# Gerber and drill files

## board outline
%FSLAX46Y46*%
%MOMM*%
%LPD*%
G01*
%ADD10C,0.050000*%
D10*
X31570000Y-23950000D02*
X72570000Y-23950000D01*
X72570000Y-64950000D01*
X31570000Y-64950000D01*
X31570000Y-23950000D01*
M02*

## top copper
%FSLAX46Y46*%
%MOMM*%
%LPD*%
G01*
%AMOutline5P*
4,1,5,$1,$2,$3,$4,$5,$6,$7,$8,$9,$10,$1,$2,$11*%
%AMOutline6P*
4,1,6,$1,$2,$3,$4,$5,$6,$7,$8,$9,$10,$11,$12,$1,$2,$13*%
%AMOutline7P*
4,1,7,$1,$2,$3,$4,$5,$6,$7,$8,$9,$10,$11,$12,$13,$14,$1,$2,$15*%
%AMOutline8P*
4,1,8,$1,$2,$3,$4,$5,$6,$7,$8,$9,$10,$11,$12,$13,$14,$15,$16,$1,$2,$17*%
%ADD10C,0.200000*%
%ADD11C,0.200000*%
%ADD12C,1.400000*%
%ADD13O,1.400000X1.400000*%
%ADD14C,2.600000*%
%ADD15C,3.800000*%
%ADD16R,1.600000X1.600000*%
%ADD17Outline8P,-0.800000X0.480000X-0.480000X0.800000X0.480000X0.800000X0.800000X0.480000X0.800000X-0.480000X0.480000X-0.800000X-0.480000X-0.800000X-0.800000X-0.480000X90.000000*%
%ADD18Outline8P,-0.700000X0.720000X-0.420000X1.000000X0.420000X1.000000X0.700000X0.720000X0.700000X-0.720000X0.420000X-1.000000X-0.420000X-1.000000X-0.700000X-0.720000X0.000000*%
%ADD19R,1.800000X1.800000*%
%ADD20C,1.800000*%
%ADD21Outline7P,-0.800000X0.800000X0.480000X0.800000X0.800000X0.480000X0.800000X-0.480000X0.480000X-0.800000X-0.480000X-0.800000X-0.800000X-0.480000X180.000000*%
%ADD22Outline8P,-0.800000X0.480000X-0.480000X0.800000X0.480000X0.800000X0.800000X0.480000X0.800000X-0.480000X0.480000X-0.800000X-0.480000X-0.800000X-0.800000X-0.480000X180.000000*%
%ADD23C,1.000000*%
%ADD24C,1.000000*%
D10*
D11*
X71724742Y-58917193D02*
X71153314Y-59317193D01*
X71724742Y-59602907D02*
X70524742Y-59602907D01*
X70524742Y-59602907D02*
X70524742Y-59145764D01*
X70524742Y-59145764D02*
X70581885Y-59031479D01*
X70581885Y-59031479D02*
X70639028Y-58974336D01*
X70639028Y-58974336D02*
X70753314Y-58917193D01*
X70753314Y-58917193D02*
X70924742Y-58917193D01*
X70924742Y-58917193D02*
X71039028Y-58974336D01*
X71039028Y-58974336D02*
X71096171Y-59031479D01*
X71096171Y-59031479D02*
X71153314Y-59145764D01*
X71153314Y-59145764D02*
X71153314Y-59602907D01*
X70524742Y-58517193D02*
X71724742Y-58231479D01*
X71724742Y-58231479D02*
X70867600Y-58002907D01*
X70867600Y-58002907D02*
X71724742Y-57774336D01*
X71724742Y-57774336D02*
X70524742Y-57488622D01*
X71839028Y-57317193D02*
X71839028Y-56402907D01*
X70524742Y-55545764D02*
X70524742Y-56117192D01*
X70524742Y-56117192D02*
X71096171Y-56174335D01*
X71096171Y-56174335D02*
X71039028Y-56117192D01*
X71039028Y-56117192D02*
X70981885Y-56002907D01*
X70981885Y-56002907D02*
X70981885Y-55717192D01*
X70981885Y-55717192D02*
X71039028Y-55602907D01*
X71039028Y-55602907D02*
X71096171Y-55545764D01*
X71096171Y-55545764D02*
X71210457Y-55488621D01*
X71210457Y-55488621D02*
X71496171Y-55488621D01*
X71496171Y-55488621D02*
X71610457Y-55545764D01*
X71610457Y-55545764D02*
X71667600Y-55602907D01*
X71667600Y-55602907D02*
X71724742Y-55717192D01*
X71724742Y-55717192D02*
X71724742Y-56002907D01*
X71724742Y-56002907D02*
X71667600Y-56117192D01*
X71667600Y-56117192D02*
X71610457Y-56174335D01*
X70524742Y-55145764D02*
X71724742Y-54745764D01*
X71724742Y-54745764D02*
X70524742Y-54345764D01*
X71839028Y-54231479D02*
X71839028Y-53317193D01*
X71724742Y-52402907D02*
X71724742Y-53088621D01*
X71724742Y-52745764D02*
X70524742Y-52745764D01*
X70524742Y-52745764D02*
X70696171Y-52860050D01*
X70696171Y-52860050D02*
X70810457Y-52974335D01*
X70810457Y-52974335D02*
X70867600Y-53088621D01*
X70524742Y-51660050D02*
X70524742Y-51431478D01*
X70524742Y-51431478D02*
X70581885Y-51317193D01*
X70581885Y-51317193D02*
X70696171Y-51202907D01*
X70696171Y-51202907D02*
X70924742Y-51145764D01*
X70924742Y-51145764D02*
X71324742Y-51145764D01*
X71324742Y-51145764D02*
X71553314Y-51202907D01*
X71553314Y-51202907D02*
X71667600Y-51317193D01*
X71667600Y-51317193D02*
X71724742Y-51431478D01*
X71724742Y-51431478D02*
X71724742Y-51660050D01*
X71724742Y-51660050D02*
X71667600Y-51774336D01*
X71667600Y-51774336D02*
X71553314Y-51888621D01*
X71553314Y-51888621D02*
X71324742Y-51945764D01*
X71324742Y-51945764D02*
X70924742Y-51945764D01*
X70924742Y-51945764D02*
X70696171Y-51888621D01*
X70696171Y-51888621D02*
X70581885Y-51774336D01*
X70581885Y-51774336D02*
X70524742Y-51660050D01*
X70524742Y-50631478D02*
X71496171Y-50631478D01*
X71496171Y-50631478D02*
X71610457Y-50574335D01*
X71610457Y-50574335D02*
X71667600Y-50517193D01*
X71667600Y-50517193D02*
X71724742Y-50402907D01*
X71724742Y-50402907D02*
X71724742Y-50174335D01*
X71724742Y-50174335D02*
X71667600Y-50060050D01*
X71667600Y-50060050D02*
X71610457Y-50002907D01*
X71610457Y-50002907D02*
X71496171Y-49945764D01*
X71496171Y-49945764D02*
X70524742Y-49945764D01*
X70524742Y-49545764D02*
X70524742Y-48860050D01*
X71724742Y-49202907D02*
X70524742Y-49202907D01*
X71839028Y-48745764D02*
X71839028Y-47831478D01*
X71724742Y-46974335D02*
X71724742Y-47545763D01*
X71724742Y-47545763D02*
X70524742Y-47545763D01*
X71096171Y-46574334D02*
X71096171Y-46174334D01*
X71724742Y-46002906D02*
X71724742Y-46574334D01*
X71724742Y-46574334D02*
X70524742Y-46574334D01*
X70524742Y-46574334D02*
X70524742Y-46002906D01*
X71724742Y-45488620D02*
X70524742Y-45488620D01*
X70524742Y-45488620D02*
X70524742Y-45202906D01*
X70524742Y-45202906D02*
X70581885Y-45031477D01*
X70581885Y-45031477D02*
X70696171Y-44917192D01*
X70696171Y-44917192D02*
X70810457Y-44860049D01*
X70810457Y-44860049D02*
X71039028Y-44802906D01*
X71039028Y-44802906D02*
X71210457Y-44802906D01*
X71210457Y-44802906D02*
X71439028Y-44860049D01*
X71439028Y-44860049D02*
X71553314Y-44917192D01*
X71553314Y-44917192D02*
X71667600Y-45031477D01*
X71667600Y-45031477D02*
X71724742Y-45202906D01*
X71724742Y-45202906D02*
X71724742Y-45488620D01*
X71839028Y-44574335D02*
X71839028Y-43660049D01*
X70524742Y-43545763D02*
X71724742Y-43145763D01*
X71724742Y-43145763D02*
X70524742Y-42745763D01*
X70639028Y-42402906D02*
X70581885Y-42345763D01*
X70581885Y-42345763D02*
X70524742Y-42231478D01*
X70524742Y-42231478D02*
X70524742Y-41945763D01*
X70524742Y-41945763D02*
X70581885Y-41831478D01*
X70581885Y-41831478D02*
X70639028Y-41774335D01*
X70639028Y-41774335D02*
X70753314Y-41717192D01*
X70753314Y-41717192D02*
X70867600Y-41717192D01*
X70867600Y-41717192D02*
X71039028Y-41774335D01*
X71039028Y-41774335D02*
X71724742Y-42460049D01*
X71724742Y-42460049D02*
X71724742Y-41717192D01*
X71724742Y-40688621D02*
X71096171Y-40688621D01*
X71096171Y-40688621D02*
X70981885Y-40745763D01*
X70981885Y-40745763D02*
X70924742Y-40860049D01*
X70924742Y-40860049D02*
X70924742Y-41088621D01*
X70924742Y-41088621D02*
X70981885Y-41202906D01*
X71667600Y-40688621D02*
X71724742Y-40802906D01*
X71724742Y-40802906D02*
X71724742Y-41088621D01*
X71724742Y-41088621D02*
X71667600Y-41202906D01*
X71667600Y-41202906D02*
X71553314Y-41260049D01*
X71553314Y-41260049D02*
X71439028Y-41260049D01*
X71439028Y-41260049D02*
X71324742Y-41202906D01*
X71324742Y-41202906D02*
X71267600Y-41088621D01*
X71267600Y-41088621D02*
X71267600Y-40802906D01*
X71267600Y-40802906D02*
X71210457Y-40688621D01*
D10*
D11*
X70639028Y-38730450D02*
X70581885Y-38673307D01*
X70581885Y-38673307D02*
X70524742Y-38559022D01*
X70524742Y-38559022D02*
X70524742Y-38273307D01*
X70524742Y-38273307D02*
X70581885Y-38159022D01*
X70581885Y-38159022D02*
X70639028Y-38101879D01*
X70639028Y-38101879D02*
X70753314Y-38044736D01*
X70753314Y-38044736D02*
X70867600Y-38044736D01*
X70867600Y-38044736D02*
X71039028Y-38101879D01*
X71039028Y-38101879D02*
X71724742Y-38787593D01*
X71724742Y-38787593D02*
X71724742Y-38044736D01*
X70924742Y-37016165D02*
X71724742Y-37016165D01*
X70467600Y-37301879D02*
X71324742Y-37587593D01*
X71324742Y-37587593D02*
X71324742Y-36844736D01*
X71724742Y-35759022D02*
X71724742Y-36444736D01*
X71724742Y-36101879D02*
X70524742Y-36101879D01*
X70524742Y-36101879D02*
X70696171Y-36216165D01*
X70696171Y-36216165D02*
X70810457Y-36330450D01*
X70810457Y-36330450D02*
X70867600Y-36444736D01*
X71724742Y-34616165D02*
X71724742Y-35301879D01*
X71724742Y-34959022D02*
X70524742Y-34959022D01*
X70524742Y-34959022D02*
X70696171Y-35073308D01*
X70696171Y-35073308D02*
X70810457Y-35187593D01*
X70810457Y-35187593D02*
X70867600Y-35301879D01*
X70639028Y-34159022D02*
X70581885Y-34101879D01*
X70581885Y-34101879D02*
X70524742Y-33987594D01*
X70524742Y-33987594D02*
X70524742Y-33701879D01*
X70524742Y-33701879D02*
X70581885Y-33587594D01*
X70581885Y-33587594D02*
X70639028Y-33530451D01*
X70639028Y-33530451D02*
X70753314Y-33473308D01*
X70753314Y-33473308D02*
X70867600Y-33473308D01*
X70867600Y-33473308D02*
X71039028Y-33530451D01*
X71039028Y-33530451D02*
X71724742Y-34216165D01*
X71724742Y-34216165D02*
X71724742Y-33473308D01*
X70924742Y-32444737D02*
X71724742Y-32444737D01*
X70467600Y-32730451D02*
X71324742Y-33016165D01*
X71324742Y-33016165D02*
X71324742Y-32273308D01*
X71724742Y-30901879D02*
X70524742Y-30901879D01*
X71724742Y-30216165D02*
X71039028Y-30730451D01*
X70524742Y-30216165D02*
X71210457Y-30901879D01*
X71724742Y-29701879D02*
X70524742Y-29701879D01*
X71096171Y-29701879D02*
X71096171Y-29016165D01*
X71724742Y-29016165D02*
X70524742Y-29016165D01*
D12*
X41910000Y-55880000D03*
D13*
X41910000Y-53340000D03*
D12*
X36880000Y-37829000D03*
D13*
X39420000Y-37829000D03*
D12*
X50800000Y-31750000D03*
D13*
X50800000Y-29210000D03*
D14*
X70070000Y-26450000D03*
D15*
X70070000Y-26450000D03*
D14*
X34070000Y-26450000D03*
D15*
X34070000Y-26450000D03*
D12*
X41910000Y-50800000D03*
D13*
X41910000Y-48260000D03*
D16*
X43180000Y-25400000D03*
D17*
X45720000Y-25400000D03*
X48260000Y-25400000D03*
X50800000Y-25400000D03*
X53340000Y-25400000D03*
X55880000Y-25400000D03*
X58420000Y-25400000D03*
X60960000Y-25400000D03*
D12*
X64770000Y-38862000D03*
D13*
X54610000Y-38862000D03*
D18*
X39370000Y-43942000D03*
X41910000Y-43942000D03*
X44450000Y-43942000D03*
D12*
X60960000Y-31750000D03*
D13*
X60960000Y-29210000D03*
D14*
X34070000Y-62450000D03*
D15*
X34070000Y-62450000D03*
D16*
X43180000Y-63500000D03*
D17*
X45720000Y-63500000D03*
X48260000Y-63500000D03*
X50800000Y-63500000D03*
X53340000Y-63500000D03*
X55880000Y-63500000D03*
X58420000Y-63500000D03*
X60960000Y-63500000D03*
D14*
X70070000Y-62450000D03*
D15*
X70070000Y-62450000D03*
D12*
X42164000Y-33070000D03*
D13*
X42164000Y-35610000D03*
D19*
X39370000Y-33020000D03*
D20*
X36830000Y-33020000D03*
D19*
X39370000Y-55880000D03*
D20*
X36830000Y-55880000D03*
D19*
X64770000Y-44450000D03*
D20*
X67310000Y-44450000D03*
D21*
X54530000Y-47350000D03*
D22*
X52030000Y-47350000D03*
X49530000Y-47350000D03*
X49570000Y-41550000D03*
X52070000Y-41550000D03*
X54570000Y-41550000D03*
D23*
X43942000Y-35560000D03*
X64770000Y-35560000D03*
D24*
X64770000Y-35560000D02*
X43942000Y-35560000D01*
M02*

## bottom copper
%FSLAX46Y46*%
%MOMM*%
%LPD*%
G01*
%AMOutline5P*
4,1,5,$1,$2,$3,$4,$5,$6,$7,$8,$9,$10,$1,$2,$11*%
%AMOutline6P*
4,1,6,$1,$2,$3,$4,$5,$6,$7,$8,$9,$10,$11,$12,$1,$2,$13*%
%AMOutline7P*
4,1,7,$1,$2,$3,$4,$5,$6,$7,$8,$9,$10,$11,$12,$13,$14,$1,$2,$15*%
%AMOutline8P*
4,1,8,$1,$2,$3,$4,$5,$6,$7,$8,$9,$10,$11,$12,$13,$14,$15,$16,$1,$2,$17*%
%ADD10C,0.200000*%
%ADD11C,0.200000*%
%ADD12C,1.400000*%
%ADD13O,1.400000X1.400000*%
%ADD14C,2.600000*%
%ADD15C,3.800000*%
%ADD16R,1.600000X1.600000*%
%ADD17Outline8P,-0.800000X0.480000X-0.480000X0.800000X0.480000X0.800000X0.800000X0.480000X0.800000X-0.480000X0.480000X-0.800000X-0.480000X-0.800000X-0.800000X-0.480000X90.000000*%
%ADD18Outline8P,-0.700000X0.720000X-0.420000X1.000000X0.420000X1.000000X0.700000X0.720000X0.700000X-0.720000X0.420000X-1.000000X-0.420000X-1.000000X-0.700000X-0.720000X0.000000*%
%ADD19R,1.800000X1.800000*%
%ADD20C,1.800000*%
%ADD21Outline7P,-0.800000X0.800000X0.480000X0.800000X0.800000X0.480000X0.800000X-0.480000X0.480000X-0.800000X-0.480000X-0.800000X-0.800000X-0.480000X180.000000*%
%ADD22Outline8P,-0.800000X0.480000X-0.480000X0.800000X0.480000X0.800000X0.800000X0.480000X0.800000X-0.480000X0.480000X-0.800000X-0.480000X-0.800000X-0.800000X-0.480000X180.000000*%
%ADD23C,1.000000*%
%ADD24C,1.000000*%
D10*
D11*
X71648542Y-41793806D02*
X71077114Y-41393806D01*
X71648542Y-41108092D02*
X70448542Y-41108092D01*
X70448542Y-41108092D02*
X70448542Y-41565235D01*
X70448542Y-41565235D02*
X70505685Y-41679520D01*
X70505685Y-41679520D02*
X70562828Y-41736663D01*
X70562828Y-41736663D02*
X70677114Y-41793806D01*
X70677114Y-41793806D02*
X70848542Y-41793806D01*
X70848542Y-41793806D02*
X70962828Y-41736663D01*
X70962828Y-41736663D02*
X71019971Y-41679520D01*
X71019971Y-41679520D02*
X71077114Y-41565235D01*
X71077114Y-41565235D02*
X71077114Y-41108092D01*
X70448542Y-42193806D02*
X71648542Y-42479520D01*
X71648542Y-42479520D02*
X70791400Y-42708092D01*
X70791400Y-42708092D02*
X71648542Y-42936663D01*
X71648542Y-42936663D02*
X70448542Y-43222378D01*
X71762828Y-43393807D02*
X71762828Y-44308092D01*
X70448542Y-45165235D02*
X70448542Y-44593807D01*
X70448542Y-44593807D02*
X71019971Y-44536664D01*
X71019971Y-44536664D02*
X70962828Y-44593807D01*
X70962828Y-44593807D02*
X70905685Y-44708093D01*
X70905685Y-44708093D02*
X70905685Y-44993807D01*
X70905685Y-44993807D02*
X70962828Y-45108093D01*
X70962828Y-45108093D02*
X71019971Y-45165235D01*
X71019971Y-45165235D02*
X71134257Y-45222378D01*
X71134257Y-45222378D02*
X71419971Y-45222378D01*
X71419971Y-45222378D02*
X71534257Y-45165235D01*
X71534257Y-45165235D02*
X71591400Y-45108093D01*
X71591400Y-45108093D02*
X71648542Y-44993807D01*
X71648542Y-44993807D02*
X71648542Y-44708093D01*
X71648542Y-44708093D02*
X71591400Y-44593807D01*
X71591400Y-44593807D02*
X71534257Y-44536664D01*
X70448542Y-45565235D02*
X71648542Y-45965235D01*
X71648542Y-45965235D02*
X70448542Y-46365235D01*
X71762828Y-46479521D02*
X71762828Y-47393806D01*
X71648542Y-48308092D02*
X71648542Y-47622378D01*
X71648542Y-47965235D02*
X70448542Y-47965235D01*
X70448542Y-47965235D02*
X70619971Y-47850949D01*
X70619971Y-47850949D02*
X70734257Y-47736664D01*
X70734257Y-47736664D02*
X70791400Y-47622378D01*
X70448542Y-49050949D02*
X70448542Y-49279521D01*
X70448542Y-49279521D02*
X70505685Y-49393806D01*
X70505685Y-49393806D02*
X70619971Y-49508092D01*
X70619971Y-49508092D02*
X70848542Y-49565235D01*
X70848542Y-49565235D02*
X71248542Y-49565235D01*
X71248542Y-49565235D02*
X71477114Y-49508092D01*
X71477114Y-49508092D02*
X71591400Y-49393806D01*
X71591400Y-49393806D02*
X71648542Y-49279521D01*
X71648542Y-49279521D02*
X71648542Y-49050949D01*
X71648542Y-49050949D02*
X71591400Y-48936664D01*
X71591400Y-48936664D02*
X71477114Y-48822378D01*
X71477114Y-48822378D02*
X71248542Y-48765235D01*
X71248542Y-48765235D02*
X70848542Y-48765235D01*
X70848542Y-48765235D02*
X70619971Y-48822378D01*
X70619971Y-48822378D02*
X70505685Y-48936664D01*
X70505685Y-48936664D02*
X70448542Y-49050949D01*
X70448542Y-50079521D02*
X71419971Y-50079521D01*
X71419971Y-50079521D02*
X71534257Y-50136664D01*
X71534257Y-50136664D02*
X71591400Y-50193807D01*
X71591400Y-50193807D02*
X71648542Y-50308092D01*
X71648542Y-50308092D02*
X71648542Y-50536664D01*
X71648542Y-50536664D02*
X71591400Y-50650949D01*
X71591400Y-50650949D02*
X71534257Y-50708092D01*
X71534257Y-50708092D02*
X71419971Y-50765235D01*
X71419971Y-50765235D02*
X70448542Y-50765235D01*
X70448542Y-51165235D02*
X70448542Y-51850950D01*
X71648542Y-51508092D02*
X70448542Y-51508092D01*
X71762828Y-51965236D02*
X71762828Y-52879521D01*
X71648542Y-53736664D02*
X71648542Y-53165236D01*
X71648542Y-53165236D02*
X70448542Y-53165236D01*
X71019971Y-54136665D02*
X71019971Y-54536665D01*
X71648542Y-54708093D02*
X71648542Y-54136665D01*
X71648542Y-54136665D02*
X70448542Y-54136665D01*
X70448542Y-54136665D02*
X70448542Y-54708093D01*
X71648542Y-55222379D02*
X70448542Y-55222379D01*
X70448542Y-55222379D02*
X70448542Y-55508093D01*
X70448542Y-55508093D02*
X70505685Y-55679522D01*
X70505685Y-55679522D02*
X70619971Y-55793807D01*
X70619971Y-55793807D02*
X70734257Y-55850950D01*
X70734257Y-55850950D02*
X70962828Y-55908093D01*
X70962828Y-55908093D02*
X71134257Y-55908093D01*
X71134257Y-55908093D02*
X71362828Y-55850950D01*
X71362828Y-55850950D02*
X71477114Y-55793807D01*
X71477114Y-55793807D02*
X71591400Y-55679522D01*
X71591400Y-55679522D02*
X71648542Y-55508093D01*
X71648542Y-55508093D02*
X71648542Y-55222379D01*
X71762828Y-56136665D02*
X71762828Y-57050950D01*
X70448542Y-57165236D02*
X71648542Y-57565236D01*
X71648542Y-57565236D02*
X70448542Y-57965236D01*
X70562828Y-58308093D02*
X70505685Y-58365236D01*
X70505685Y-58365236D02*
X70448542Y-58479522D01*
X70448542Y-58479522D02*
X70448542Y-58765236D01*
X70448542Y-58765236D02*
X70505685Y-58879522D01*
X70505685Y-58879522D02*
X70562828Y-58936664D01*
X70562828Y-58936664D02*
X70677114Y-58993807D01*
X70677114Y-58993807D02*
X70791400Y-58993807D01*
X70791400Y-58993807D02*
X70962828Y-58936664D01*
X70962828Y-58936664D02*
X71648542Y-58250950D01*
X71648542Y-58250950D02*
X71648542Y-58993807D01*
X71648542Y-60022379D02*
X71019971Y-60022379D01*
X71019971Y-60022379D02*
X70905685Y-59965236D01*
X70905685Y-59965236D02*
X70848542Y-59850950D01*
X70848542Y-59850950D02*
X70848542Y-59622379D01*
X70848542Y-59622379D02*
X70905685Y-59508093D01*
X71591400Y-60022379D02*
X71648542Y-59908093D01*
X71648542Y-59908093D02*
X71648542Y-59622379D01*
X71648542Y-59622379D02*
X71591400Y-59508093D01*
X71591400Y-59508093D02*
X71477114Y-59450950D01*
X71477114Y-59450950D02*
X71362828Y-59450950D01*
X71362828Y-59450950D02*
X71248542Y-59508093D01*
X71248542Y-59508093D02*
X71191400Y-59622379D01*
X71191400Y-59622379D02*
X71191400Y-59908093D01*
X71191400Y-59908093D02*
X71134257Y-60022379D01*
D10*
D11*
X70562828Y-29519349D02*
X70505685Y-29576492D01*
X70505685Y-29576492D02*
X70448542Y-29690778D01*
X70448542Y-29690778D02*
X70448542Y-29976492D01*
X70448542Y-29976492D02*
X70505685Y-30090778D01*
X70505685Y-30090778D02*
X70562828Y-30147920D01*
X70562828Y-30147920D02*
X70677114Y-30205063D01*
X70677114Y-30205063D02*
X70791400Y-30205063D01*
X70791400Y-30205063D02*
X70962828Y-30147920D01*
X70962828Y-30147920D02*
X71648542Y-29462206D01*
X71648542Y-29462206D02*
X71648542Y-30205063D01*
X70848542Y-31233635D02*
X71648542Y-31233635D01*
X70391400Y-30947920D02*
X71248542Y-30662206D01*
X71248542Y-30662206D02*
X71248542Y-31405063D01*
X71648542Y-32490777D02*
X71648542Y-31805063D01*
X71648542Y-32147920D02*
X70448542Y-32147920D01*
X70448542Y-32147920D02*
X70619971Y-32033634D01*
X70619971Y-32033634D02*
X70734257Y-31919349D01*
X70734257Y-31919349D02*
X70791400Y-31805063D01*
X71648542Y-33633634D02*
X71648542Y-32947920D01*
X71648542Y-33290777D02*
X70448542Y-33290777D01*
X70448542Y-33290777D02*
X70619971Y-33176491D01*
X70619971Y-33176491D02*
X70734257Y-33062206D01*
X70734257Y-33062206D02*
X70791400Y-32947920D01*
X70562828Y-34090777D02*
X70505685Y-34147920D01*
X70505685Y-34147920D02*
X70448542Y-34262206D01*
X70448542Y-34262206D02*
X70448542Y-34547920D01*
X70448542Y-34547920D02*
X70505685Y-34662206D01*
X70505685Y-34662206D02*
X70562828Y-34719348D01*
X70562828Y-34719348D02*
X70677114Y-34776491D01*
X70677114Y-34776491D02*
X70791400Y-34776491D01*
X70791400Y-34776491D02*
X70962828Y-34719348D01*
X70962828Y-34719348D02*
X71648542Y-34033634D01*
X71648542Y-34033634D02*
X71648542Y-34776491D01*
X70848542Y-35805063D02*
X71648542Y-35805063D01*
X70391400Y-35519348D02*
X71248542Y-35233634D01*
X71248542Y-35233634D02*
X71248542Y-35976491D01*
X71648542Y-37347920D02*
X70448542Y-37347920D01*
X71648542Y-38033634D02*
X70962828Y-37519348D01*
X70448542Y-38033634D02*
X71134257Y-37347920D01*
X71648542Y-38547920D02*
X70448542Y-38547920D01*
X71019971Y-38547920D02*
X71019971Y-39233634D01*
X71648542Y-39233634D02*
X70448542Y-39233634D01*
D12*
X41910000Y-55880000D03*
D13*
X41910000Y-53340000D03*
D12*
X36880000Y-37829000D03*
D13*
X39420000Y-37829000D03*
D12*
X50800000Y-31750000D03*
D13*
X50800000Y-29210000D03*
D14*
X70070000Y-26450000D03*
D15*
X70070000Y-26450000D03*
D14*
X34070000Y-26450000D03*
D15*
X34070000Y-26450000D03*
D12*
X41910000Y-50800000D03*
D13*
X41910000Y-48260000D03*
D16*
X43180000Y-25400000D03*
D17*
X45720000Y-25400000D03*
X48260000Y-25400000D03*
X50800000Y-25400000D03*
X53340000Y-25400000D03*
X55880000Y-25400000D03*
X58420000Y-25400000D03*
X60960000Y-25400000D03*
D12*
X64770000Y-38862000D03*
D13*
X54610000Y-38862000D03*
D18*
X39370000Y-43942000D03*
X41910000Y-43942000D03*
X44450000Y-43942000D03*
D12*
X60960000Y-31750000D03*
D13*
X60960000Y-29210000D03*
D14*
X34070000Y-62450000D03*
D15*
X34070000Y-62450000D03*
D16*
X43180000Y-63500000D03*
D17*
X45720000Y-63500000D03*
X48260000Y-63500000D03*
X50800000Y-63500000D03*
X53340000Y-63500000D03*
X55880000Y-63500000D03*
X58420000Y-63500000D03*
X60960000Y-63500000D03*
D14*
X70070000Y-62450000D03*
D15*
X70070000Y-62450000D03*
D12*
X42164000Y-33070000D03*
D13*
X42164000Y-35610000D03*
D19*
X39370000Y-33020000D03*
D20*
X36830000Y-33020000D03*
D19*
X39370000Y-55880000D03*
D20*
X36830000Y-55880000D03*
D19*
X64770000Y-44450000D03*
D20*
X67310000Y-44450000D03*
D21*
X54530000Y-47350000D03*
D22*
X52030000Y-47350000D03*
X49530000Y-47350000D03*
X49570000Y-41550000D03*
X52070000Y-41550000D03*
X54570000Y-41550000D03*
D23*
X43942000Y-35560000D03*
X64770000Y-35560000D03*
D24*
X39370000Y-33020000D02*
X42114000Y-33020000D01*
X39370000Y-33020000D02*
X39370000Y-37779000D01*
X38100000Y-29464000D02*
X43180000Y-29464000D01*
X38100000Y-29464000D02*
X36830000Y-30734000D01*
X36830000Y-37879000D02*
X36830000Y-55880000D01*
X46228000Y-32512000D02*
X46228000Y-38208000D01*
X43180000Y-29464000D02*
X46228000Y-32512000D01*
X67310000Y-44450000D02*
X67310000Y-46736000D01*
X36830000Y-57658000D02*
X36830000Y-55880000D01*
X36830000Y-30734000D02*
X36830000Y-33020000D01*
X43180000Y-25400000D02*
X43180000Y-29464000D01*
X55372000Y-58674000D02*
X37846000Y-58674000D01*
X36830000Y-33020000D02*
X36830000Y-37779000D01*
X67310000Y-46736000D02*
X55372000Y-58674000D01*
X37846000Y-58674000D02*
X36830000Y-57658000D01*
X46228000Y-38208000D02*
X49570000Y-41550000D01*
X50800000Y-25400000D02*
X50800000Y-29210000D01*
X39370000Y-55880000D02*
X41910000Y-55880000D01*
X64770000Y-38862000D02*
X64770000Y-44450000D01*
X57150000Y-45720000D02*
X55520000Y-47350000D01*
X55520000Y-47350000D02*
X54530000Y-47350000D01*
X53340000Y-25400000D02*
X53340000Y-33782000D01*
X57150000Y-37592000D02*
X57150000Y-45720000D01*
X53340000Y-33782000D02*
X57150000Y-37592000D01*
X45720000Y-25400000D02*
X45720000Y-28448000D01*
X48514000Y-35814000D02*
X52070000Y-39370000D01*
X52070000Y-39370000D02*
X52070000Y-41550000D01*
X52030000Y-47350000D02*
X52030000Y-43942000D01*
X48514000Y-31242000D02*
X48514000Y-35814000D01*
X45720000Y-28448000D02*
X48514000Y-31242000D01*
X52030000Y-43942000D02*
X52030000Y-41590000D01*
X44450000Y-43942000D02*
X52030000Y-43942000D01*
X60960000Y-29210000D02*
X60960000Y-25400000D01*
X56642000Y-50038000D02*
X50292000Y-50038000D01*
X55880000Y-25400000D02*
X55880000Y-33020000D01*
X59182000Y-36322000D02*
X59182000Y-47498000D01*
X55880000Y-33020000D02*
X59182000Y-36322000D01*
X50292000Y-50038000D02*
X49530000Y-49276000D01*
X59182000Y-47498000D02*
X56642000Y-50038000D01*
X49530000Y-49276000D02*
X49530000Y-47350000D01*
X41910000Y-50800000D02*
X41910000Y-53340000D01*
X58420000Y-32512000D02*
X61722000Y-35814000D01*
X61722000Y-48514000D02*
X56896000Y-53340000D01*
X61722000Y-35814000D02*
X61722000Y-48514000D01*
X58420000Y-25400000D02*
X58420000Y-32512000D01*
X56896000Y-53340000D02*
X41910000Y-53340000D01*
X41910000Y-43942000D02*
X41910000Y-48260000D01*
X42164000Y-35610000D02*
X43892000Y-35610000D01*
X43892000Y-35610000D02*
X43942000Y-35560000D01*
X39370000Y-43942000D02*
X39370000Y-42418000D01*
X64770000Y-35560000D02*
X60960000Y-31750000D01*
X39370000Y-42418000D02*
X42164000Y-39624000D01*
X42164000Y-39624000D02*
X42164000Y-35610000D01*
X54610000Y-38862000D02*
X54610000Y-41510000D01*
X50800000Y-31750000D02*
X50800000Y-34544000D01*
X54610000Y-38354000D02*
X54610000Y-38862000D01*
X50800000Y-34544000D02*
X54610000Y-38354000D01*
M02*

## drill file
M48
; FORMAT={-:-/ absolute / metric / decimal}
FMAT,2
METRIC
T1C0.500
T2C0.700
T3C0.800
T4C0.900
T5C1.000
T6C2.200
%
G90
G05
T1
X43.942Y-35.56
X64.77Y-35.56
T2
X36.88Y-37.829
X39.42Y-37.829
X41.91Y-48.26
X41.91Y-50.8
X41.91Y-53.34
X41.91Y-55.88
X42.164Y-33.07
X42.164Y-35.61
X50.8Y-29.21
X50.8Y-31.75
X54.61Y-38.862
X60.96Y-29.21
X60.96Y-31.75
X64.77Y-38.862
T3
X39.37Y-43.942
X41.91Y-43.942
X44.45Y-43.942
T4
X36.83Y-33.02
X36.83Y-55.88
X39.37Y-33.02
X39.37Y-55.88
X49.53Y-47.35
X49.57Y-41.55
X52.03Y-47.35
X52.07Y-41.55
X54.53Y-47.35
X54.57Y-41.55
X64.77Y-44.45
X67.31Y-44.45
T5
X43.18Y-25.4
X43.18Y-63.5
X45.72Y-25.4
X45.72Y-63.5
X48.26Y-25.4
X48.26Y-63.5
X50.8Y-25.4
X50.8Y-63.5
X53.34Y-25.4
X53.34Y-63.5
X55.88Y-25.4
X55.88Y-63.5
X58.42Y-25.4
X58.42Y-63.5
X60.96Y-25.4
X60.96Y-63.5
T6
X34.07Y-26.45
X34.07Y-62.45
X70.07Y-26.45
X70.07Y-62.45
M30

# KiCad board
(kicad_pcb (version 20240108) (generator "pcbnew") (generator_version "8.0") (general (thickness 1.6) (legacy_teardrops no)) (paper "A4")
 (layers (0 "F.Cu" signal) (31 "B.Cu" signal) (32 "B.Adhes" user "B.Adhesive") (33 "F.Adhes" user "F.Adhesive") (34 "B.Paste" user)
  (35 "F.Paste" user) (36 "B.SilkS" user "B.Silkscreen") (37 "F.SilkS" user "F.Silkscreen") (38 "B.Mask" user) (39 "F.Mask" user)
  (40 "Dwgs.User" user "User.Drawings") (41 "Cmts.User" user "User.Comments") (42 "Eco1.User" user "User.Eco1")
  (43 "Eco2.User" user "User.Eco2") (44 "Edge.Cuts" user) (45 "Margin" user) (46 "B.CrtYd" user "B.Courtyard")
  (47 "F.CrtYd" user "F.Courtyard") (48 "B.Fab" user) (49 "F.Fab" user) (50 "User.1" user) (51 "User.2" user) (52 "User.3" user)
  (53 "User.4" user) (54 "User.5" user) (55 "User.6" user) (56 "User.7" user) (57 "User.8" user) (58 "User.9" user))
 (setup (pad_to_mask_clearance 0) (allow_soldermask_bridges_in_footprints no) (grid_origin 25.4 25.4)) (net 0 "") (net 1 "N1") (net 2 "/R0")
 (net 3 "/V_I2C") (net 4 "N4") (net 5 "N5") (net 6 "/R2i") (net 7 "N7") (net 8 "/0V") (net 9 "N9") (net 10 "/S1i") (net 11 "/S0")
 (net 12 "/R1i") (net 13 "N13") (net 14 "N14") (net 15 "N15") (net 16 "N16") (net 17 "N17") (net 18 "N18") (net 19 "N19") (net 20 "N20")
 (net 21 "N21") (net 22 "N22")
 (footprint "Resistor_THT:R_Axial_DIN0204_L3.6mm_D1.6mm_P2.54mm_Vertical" (layer "F.Cu") (at 41.91 55.88 90)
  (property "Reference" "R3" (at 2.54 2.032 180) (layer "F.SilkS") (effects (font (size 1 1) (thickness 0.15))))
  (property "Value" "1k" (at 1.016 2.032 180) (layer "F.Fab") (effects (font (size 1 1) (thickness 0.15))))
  (pad "1" thru_hole circle (at 0 0 90) (size 1.4 1.4) (drill 0.7) (layers "*.Cu" "*.Mask") (remove_unused_layers no) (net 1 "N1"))
  (pad "2" thru_hole oval (at 2.54 0 90) (size 1.4 1.4) (drill 0.7) (layers "*.Cu" "*.Mask") (remove_unused_layers no) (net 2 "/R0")))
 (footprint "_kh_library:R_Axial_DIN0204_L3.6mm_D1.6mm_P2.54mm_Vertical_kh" (layer "F.Cu") (at 36.88 37.829)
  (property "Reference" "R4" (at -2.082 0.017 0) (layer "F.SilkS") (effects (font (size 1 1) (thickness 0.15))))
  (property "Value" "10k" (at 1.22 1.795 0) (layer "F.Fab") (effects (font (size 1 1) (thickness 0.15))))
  (pad "1" thru_hole circle (at 0 0) (size 1.4 1.4) (drill 0.7) (layers "*.Cu" "*.Mask") (remove_unused_layers no) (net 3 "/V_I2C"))
  (pad "2" thru_hole oval (at 2.54 0) (size 1.4 1.4) (drill 0.7) (layers "*.Cu" "*.Mask") (remove_unused_layers no) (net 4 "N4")))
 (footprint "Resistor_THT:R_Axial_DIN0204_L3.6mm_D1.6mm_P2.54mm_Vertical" (layer "F.Cu") (at 50.8 31.75 90)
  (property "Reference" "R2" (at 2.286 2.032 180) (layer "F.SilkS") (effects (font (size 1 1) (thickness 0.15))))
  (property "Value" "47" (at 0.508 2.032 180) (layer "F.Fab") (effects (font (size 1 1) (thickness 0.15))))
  (pad "1" thru_hole circle (at 0 0 90) (size 1.4 1.4) (drill 0.7) (layers "*.Cu" "*.Mask") (remove_unused_layers no) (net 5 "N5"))
  (pad "2" thru_hole oval (at 2.54 0 90) (size 1.4 1.4) (drill 0.7) (layers "*.Cu" "*.Mask") (remove_unused_layers no) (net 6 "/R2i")))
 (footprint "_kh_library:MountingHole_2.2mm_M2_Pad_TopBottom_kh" (layer "F.Cu") (at 70.07 26.45)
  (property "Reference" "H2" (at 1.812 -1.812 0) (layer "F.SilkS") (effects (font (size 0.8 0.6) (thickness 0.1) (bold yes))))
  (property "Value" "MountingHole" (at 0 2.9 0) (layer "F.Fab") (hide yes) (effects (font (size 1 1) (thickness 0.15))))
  (pad "1" thru_hole circle (at 0 0) (size 2.6 2.6) (drill 2.2) (layers "*.Cu" "*.Mask") (remove_unused_layers no))
  (pad "1" connect circle (at 0 0) (size 3.8 3.8) (layers "F.Cu" "F.Mask"))
  (pad "1" connect circle (at 0 0) (size 3.8 3.8) (layers "B.Cu" "B.Mask")))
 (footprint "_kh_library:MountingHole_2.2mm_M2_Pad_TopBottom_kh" (layer "F.Cu") (at 34.07 26.45)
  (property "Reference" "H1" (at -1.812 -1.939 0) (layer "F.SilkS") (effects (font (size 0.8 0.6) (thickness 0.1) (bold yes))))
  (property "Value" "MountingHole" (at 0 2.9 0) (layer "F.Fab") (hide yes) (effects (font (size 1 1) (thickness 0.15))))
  (pad "1" thru_hole circle (at 0 0) (size 2.6 2.6) (drill 2.2) (layers "*.Cu" "*.Mask") (remove_unused_layers no))
  (pad "1" connect circle (at 0 0) (size 3.8 3.8) (layers "F.Cu" "F.Mask"))
  (pad "1" connect circle (at 0 0) (size 3.8 3.8) (layers "B.Cu" "B.Mask")))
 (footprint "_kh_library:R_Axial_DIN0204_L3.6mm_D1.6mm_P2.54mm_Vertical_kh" (layer "F.Cu") (at 41.91 50.8 90)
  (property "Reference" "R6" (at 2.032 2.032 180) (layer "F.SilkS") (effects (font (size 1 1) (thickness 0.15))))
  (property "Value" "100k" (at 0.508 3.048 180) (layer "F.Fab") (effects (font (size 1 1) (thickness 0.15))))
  (pad "1" thru_hole circle (at 0 0 90) (size 1.4 1.4) (drill 0.7) (layers "*.Cu" "*.Mask") (remove_unused_layers no) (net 2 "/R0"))
  (pad "2" thru_hole oval (at 2.54 0 90) (size 1.4 1.4) (drill 0.7) (layers "*.Cu" "*.Mask") (remove_unused_layers no) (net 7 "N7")))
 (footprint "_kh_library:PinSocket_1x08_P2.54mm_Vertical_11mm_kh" (layer "F.Cu") (at 43.18 25.4 90)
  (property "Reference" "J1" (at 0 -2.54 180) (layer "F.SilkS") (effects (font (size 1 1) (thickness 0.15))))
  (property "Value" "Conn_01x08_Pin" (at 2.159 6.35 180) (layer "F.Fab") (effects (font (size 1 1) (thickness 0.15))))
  (pad "1" thru_hole rect (at 0 0 90) (size 1.6 1.6) (drill 1) (layers "*.Cu" "*.Mask") (remove_unused_layers no) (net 3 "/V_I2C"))
  (pad "2" thru_hole roundrect (at 0 2.54 90) (size 1.6 1.6) (drill 1) (layers "*.Cu" "*.Mask") (remove_unused_layers no)
   (roundrect_rratio 0) (chamfer_ratio 0.2) (chamfer top_left top_right bottom_left bottom_right) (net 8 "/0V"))
  (pad "3" thru_hole roundrect (at 0 5.08 90) (size 1.6 1.6) (drill 1) (layers "*.Cu" "*.Mask") (remove_unused_layers no)
   (roundrect_rratio 0) (chamfer_ratio 0.2) (chamfer top_left top_right bottom_left bottom_right) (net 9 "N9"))
  (pad "4" thru_hole roundrect (at 0 7.62 90) (size 1.6 1.6) (drill 1) (layers "*.Cu" "*.Mask") (remove_unused_layers no)
   (roundrect_rratio 0) (chamfer_ratio 0.2) (chamfer top_left top_right bottom_left bottom_right) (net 6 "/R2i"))
  (pad "5" thru_hole roundrect (at 0 10.16 90) (size 1.6 1.6) (drill 1) (layers "*.Cu" "*.Mask") (remove_unused_layers no)
   (roundrect_rratio 0) (chamfer_ratio 0.2) (chamfer top_left top_right bottom_left bottom_right) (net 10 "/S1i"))
  (pad "6" thru_hole roundrect (at 0 12.7 90) (size 1.6 1.6) (drill 1) (layers "*.Cu" "*.Mask") (remove_unused_layers no)
   (roundrect_rratio 0) (chamfer_ratio 0.2) (chamfer top_left top_right bottom_left bottom_right) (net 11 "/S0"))
  (pad "7" thru_hole roundrect (at 0 15.24 90) (size 1.6 1.6) (drill 1) (layers "*.Cu" "*.Mask") (remove_unused_layers no)
   (roundrect_rratio 0) (chamfer_ratio 0.2) (chamfer top_left top_right bottom_left bottom_right) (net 2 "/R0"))
  (pad "8" thru_hole roundrect (at 0 17.78 90) (size 1.6 1.6) (drill 1) (layers "*.Cu" "*.Mask") (remove_unused_layers no)
   (roundrect_rratio 0) (chamfer_ratio 0.2) (chamfer top_left top_right bottom_left bottom_right) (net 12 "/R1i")))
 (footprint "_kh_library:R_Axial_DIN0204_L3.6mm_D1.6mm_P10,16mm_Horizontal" (layer "F.Cu") (at 64.77 38.862 180)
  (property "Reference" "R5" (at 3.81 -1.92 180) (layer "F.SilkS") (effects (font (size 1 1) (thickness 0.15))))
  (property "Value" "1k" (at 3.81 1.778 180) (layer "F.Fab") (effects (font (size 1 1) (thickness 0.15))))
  (pad "1" thru_hole circle (at 0 0 180) (size 1.4 1.4) (drill 0.7) (layers "*.Cu" "*.Mask") (remove_unused_layers no) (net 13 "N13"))
  (pad "2" thru_hole oval (at 10.16 0 180) (size 1.4 1.4) (drill 0.7) (layers "*.Cu" "*.Mask") (remove_unused_layers no) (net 5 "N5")))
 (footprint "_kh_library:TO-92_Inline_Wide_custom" (layer "F.Cu") (at 39.37 43.942)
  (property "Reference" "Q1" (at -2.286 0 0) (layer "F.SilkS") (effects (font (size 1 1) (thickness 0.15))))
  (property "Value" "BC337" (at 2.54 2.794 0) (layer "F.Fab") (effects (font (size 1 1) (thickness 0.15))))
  (pad "1" thru_hole roundrect (at 0 0) (size 1.4 2) (drill 0.8) (layers "*.Cu" "*.Mask") (remove_unused_layers no) (roundrect_rratio 0)
   (chamfer_ratio 0.2) (chamfer top_left top_right bottom_left bottom_right) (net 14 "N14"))
  (pad "2" thru_hole roundrect (at 2.54 0) (size 1.4 2) (drill 0.8) (layers "*.Cu" "*.Mask") (remove_unused_layers no) (roundrect_rratio 0)
   (chamfer_ratio 0.2) (chamfer top_left top_right bottom_left bottom_right) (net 7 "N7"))
  (pad "3" thru_hole roundrect (at 5.08 0) (size 1.4 2) (drill 0.8) (layers "*.Cu" "*.Mask") (remove_unused_layers no) (roundrect_rratio 0)
   (chamfer_ratio 0.2) (chamfer top_left top_right bottom_left bottom_right) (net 8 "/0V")))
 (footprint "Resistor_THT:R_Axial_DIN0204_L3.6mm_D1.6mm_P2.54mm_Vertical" (layer "F.Cu") (at 60.96 31.75 90)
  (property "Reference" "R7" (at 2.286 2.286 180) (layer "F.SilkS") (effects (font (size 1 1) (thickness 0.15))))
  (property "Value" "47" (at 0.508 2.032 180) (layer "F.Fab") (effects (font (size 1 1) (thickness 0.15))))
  (pad "1" thru_hole circle (at 0 0 90) (size 1.4 1.4) (drill 0.7) (layers "*.Cu" "*.Mask") (remove_unused_layers no) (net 14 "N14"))
  (pad "2" thru_hole oval (at 2.54 0 90) (size 1.4 1.4) (drill 0.7) (layers "*.Cu" "*.Mask") (remove_unused_layers no) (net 12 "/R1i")))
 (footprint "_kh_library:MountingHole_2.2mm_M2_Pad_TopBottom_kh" (layer "F.Cu") (at 34.07 62.45)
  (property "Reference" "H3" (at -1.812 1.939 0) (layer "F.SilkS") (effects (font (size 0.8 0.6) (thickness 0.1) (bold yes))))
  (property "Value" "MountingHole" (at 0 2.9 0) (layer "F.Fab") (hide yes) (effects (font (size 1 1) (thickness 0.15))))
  (pad "1" thru_hole circle (at 0 0) (size 2.6 2.6) (drill 2.2) (layers "*.Cu" "*.Mask") (remove_unused_layers no))
  (pad "1" connect circle (at 0 0) (size 3.8 3.8) (layers "F.Cu" "F.Mask"))
  (pad "1" connect circle (at 0 0) (size 3.8 3.8) (layers "B.Cu" "B.Mask")))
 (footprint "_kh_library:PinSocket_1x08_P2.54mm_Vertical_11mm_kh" (layer "F.Cu") (at 43.18 63.5 90)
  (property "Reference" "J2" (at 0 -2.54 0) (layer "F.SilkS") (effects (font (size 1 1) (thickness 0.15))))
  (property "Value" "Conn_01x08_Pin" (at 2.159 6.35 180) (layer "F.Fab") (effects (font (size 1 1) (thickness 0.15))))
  (pad "1" thru_hole rect (at 0 0 90) (size 1.6 1.6) (drill 1) (layers "*.Cu" "*.Mask") (remove_unused_layers no) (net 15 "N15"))
  (pad "2" thru_hole roundrect (at 0 2.54 90) (size 1.6 1.6) (drill 1) (layers "*.Cu" "*.Mask") (remove_unused_layers no)
   (roundrect_rratio 0) (chamfer_ratio 0.2) (chamfer top_left top_right bottom_left bottom_right) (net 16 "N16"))
  (pad "3" thru_hole roundrect (at 0 5.08 90) (size 1.6 1.6) (drill 1) (layers "*.Cu" "*.Mask") (remove_unused_layers no)
   (roundrect_rratio 0) (chamfer_ratio 0.2) (chamfer top_left top_right bottom_left bottom_right) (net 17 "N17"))
  (pad "4" thru_hole roundrect (at 0 7.62 90) (size 1.6 1.6) (drill 1) (layers "*.Cu" "*.Mask") (remove_unused_layers no)
   (roundrect_rratio 0) (chamfer_ratio 0.2) (chamfer top_left top_right bottom_left bottom_right) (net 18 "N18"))
  (pad "5" thru_hole roundrect (at 0 10.16 90) (size 1.6 1.6) (drill 1) (layers "*.Cu" "*.Mask") (remove_unused_layers no)
   (roundrect_rratio 0) (chamfer_ratio 0.2) (chamfer top_left top_right bottom_left bottom_right) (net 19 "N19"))
  (pad "6" thru_hole roundrect (at 0 12.7 90) (size 1.6 1.6) (drill 1) (layers "*.Cu" "*.Mask") (remove_unused_layers no)
   (roundrect_rratio 0) (chamfer_ratio 0.2) (chamfer top_left top_right bottom_left bottom_right) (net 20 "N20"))
  (pad "7" thru_hole roundrect (at 0 15.24 90) (size 1.6 1.6) (drill 1) (layers "*.Cu" "*.Mask") (remove_unused_layers no)
   (roundrect_rratio 0) (chamfer_ratio 0.2) (chamfer top_left top_right bottom_left bottom_right) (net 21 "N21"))
  (pad "8" thru_hole roundrect (at 0 17.78 90) (size 1.6 1.6) (drill 1) (layers "*.Cu" "*.Mask") (remove_unused_layers no)
   (roundrect_rratio 0) (chamfer_ratio 0.2) (chamfer top_left top_right bottom_left bottom_right) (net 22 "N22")))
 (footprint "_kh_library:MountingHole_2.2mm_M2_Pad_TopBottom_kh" (layer "F.Cu") (at 70.07 62.45)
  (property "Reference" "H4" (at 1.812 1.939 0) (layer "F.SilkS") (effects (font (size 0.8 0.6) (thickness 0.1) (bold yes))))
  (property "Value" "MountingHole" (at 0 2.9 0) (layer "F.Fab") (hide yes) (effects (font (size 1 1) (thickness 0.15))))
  (pad "1" thru_hole circle (at 0 0) (size 2.6 2.6) (drill 2.2) (layers "*.Cu" "*.Mask") (remove_unused_layers no))
  (pad "1" connect circle (at 0 0) (size 3.8 3.8) (layers "F.Cu" "F.Mask"))
  (pad "1" connect circle (at 0 0) (size 3.8 3.8) (layers "B.Cu" "B.Mask")))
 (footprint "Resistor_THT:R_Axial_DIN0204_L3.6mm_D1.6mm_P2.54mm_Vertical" (layer "F.Cu") (at 42.164 33.07 -90)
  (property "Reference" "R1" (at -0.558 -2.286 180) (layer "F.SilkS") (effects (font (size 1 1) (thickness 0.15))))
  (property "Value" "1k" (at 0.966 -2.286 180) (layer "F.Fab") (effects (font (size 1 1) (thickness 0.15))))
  (pad "1" thru_hole circle (at 0 0 270) (size 1.4 1.4) (drill 0.7) (layers "*.Cu" "*.Mask") (remove_unused_layers no) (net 4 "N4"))
  (pad "2" thru_hole oval (at 2.54 0 270) (size 1.4 1.4) (drill 0.7) (layers "*.Cu" "*.Mask") (remove_unused_layers no) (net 14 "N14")))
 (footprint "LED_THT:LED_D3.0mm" (layer "B.Cu") (at 39.37 33.02 180)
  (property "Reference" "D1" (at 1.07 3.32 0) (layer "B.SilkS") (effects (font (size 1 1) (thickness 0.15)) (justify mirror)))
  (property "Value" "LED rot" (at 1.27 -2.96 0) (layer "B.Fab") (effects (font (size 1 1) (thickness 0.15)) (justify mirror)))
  (pad "1" thru_hole rect (at 0 0 180) (size 1.8 1.8) (drill 0.9) (layers "*.Cu" "*.Mask") (remove_unused_layers no) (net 4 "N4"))
  (pad "2" thru_hole circle (at 2.54 0 180) (size 1.8 1.8) (drill 0.9) (layers "*.Cu" "*.Mask") (remove_unused_layers no) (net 3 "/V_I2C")))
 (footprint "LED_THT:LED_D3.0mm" (layer "B.Cu") (at 39.37 55.88 180)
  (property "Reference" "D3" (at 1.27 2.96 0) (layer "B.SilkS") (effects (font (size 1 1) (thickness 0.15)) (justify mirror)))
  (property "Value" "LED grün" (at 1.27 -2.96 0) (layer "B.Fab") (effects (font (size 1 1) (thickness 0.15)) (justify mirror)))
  (pad "1" thru_hole rect (at 0 0 180) (size 1.8 1.8) (drill 0.9) (layers "*.Cu" "*.Mask") (remove_unused_layers no) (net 1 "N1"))
  (pad "2" thru_hole circle (at 2.54 0 180) (size 1.8 1.8) (drill 0.9) (layers "*.Cu" "*.Mask") (remove_unused_layers no) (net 3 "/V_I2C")))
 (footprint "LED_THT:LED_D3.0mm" (layer "B.Cu") (at 64.77 44.45)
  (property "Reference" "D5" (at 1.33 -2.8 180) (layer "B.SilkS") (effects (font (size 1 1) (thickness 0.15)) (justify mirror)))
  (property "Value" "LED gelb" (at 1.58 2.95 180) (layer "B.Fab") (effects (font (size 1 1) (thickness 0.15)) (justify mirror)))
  (pad "1" thru_hole rect (at 0 0) (size 1.8 1.8) (drill 0.9) (layers "*.Cu" "*.Mask") (remove_unused_layers no) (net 13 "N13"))
  (pad "2" thru_hole circle (at 2.54 0) (size 1.8 1.8) (drill 0.9) (layers "*.Cu" "*.Mask") (remove_unused_layers no) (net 3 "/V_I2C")))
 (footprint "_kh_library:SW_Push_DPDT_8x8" (layer "B.Cu") (at 54.57 47.35 180)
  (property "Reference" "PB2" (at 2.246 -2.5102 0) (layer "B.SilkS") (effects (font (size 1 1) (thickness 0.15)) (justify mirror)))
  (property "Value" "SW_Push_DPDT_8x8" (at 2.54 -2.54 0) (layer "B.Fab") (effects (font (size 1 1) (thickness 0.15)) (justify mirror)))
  (pad "1" thru_hole roundrect (at 0.04 0 180) (size 1.6 1.6) (drill 0.9) (layers "*.Cu" "*.Mask") (remove_unused_layers no)
   (roundrect_rratio 0) (chamfer_ratio 0.2) (chamfer top_right bottom_left bottom_right) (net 10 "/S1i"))
  (pad "2" thru_hole roundrect (at 2.54 0 180) (size 1.6 1.6) (drill 0.9) (layers "*.Cu" "*.Mask") (remove_unused_layers no)
   (roundrect_rratio 0) (chamfer_ratio 0.2) (chamfer top_left top_right bottom_left bottom_right) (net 8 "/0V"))
  (pad "3" thru_hole roundrect (at 5.04 0 180) (size 1.6 1.6) (drill 0.9) (layers "*.Cu" "*.Mask") (remove_unused_layers no)
   (roundrect_rratio 0) (chamfer_ratio 0.2) (chamfer top_left top_right bottom_left bottom_right) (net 11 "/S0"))
  (pad "4" thru_hole roundrect (at 5 5.8 180) (size 1.6 1.6) (drill 0.9) (layers "*.Cu" "*.Mask") (remove_unused_layers no)
   (roundrect_rratio 0) (chamfer_ratio 0.2) (chamfer top_left top_right bottom_left bottom_right) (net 3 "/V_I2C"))
  (pad "5" thru_hole roundrect (at 2.5 5.8 180) (size 1.6 1.6) (drill 0.9) (layers "*.Cu" "*.Mask") (remove_unused_layers no)
   (roundrect_rratio 0) (chamfer_ratio 0.2) (chamfer top_left top_right bottom_left bottom_right) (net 8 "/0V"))
  (pad "6" thru_hole roundrect (at 0 5.8 180) (size 1.6 1.6) (drill 0.9) (layers "*.Cu" "*.Mask") (remove_unused_layers no)
   (roundrect_rratio 0) (chamfer_ratio 0.2) (chamfer top_left top_right bottom_left bottom_right) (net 5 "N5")))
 (gr_rect (start 31.57 23.95) (end 72.57 64.95) (stroke (width 0.05) (type default)) (fill none) (layer "Edge.Cuts"))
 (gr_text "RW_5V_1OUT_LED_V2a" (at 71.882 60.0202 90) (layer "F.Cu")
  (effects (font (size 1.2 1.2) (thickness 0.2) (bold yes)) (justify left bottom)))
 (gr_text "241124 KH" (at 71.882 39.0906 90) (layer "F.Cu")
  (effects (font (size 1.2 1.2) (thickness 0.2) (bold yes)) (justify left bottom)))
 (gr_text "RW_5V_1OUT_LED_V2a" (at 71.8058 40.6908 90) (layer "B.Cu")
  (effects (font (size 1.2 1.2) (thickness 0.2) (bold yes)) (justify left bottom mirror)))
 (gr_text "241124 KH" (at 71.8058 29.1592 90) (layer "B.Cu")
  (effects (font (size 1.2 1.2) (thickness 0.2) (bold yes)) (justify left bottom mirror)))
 (segment (start 39.37 33.02) (end 42.114 33.02) (width 1) (layer "B.Cu") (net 4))
 (segment (start 39.37 33.02) (end 39.37 37.779) (width 1) (layer "B.Cu") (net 4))
 (segment (start 38.1 29.464) (end 43.18 29.464) (width 1) (layer "B.Cu") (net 3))
 (segment (start 38.1 29.464) (end 36.83 30.734) (width 1) (layer "B.Cu") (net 3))
 (segment (start 36.83 37.879) (end 36.83 55.88) (width 1) (layer "B.Cu") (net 3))
 (segment (start 46.228 32.512) (end 46.228 38.208) (width 1) (layer "B.Cu") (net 3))
 (segment (start 43.18 29.464) (end 46.228 32.512) (width 1) (layer "B.Cu") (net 3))
 (segment (start 67.31 44.45) (end 67.31 46.736) (width 1) (layer "B.Cu") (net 3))
 (segment (start 36.83 57.658) (end 36.83 55.88) (width 1) (layer "B.Cu") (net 3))
 (segment (start 36.83 30.734) (end 36.83 33.02) (width 1) (layer "B.Cu") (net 3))
 (segment (start 43.18 25.4) (end 43.18 29.464) (width 1) (layer "B.Cu") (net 3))
 (segment (start 55.372 58.674) (end 37.846 58.674) (width 1) (layer "B.Cu") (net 3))
 (segment (start 36.83 33.02) (end 36.83 37.779) (width 1) (layer "B.Cu") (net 3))
 (segment (start 67.31 46.736) (end 55.372 58.674) (width 1) (layer "B.Cu") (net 3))
 (segment (start 37.846 58.674) (end 36.83 57.658) (width 1) (layer "B.Cu") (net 3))
 (segment (start 46.228 38.208) (end 49.57 41.55) (width 1) (layer "B.Cu") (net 3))
 (segment (start 50.8 25.4) (end 50.8 29.21) (width 1) (layer "B.Cu") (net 6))
 (segment (start 39.37 55.88) (end 41.91 55.88) (width 1) (layer "B.Cu") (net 1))
 (segment (start 64.77 38.862) (end 64.77 44.45) (width 1) (layer "B.Cu") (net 13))
 (segment (start 57.15 45.72) (end 55.52 47.35) (width 1) (layer "B.Cu") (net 10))
 (segment (start 55.52 47.35) (end 54.53 47.35) (width 1) (layer "B.Cu") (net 10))
 (segment (start 53.34 25.4) (end 53.34 33.782) (width 1) (layer "B.Cu") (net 10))
 (segment (start 57.15 37.592) (end 57.15 45.72) (width 1) (layer "B.Cu") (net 10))
 (segment (start 53.34 33.782) (end 57.15 37.592) (width 1) (layer "B.Cu") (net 10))
 (segment (start 45.72 25.4) (end 45.72 28.448) (width 1) (layer "B.Cu") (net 8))
 (segment (start 48.514 35.814) (end 52.07 39.37) (width 1) (layer "B.Cu") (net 8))
 (segment (start 52.07 39.37) (end 52.07 41.55) (width 1) (layer "B.Cu") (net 8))
 (segment (start 52.03 47.35) (end 52.03 43.942) (width 1) (layer "B.Cu") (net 8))
 (segment (start 48.514 31.242) (end 48.514 35.814) (width 1) (layer "B.Cu") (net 8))
 (segment (start 45.72 28.448) (end 48.514 31.242) (width 1) (layer "B.Cu") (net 8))
 (segment (start 52.03 43.942) (end 52.03 41.59) (width 1) (layer "B.Cu") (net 8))
 (segment (start 44.45 43.942) (end 52.03 43.942) (width 1) (layer "B.Cu") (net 8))
 (segment (start 60.96 29.21) (end 60.96 25.4) (width 1) (layer "B.Cu") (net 12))
 (segment (start 56.642 50.038) (end 50.292 50.038) (width 1) (layer "B.Cu") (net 11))
 (segment (start 55.88 25.4) (end 55.88 33.02) (width 1) (layer "B.Cu") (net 11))
 (segment (start 59.182 36.322) (end 59.182 47.498) (width 1) (layer "B.Cu") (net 11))
 (segment (start 55.88 33.02) (end 59.182 36.322) (width 1) (layer "B.Cu") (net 11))
 (segment (start 50.292 50.038) (end 49.53 49.276) (width 1) (layer "B.Cu") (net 11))
 (segment (start 59.182 47.498) (end 56.642 50.038) (width 1) (layer "B.Cu") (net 11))
 (segment (start 49.53 49.276) (end 49.53 47.35) (width 1) (layer "B.Cu") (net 11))
 (segment (start 41.91 50.8) (end 41.91 53.34) (width 1) (layer "B.Cu") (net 2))
 (segment (start 58.42 32.512) (end 61.722 35.814) (width 1) (layer "B.Cu") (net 2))
 (segment (start 61.722 48.514) (end 56.896 53.34) (width 1) (layer "B.Cu") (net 2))
 (segment (start 61.722 35.814) (end 61.722 48.514) (width 1) (layer "B.Cu") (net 2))
 (segment (start 58.42 25.4) (end 58.42 32.512) (width 1) (layer "B.Cu") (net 2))
 (segment (start 56.896 53.34) (end 41.91 53.34) (width 1) (layer "B.Cu") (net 2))
 (segment (start 41.91 43.942) (end 41.91 48.26) (width 1) (layer "B.Cu") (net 7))
 (segment (start 64.77 35.56) (end 43.942 35.56) (width 1) (layer "F.Cu") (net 14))
 (via (at 43.942 35.56) (size 1) (drill 0.5) (layers "F.Cu" "B.Cu") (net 14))
 (via (at 64.77 35.56) (size 1) (drill 0.5) (layers "F.Cu" "B.Cu") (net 14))
 (segment (start 42.164 35.61) (end 43.892 35.61) (width 1) (layer "B.Cu") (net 14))
 (segment (start 43.892 35.61) (end 43.942 35.56) (width 1) (layer "B.Cu") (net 14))
 (segment (start 39.37 43.942) (end 39.37 42.418) (width 1) (layer "B.Cu") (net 14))
 (segment (start 64.77 35.56) (end 60.96 31.75) (width 1) (layer "B.Cu") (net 14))
 (segment (start 39.37 42.418) (end 42.164 39.624) (width 1) (layer "B.Cu") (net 14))
 (segment (start 42.164 39.624) (end 42.164 35.61) (width 1) (layer "B.Cu") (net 14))
 (segment (start 54.61 38.862) (end 54.61 41.51) (width 1) (layer "B.Cu") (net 5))
 (segment (start 50.8 31.75) (end 50.8 34.544) (width 1) (layer "B.Cu") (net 5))
 (segment (start 54.61 38.354) (end 54.61 38.862) (width 1) (layer "B.Cu") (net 5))
 (segment (start 50.8 34.544) (end 54.61 38.354) (width 1) (layer "B.Cu") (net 5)))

